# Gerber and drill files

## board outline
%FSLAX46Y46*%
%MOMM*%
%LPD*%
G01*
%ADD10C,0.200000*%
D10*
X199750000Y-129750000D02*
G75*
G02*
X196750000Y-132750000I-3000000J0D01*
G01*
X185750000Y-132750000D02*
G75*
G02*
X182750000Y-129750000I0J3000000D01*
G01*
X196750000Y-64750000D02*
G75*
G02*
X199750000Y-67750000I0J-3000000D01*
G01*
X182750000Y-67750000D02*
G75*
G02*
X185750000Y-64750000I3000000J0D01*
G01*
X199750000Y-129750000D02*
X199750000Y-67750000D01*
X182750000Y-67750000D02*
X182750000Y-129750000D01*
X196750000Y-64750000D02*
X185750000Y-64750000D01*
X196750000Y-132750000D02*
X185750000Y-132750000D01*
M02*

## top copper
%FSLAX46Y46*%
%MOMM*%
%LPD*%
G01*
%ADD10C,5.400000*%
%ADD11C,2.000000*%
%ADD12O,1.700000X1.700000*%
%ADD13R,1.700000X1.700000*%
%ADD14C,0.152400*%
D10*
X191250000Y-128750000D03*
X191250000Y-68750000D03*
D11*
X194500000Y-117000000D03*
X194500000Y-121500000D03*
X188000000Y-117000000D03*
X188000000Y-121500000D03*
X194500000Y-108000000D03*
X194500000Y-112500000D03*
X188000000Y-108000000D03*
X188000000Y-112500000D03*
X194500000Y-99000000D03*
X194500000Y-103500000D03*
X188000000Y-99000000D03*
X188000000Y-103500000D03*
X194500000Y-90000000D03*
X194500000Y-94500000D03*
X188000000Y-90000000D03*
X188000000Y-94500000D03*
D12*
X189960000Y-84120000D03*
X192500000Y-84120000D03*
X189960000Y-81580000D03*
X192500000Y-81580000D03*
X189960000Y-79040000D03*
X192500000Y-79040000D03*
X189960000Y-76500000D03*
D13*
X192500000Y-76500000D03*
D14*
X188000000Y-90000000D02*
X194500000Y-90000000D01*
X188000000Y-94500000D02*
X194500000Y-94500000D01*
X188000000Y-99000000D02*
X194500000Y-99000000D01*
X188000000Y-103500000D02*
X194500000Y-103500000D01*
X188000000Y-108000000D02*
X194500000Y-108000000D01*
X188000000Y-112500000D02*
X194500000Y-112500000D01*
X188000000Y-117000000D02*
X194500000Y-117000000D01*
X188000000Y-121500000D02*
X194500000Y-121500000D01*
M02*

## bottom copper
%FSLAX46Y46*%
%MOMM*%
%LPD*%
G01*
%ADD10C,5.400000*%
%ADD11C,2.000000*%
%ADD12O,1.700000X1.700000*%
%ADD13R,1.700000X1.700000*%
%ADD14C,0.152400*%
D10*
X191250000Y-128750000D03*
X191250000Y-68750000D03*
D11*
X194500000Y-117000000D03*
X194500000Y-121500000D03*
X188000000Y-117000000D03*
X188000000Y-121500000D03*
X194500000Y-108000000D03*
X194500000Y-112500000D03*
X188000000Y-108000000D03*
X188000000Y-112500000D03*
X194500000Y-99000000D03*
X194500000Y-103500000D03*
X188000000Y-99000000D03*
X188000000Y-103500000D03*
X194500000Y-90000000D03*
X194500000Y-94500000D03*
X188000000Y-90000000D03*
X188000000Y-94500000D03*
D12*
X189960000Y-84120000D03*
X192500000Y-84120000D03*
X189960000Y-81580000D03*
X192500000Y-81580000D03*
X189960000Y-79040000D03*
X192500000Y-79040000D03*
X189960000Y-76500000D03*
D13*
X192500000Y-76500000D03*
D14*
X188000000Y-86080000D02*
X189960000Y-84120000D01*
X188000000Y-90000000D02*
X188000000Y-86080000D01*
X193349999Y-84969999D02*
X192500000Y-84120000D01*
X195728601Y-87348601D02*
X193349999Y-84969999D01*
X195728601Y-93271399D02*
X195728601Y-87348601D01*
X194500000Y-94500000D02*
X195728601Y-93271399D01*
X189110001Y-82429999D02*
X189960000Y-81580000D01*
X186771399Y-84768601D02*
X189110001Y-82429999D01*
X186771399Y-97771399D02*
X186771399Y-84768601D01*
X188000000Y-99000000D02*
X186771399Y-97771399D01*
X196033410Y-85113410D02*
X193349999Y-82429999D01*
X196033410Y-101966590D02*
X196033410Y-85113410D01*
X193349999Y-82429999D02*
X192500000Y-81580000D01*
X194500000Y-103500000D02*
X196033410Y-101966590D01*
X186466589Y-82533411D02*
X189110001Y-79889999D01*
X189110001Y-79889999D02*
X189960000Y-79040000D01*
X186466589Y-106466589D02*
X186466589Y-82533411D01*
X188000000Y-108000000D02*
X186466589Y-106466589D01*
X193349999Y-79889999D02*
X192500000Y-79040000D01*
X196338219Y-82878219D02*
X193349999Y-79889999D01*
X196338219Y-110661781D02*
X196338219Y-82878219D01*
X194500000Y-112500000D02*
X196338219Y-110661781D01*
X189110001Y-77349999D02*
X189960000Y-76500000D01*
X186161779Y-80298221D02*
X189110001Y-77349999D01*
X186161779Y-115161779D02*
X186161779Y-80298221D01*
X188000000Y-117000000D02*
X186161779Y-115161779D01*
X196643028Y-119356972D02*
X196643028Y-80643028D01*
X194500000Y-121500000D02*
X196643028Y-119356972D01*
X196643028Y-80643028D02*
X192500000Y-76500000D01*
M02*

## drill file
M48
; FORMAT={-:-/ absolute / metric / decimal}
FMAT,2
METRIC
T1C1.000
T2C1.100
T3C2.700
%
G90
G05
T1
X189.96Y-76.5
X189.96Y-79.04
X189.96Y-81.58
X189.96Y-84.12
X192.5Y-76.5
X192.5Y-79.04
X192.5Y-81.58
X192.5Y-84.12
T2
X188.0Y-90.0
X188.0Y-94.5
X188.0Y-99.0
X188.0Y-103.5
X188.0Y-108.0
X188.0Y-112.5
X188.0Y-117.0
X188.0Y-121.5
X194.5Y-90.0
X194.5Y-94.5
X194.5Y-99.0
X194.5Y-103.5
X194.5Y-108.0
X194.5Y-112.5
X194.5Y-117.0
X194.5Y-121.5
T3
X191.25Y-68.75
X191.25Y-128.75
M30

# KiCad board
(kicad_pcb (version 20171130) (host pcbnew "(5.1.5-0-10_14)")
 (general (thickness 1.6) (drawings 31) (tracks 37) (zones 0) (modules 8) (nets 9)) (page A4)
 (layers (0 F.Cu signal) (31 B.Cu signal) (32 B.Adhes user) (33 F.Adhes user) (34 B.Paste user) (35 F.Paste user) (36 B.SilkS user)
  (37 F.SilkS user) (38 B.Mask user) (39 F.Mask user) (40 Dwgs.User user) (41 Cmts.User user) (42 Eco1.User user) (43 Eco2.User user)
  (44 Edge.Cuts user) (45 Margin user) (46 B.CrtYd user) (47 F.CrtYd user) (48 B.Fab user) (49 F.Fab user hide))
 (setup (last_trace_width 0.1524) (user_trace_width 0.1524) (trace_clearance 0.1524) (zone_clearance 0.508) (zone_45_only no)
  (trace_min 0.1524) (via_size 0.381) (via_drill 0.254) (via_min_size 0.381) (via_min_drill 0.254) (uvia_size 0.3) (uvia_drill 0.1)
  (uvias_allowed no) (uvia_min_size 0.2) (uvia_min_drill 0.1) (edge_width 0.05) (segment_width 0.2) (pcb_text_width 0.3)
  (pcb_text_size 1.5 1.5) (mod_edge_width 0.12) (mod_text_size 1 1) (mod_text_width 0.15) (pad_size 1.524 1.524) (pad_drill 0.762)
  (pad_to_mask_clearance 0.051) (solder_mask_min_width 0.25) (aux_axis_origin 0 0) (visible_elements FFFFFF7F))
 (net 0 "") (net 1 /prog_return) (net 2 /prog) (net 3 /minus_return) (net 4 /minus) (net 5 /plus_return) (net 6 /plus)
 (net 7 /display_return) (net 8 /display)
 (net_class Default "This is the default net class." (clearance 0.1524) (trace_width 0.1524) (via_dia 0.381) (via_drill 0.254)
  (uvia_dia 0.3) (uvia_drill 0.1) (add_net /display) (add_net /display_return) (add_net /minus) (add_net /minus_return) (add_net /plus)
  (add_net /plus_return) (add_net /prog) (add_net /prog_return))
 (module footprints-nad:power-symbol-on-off (layer F.Cu) (at 185.25 92.25 270)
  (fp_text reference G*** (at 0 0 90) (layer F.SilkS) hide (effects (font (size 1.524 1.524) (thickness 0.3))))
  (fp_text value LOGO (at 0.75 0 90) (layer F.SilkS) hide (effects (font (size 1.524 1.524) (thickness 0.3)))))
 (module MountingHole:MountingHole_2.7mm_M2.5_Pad (layer F.Cu) (at 191.25 128.75)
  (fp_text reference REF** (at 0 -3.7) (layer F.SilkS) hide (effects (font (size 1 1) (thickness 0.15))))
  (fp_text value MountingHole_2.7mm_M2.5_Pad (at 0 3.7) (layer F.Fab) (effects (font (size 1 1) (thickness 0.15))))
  (pad 1 thru_hole circle (at 0 0) (size 5.4 5.4) (drill 2.7) (layers *.Cu *.Mask)))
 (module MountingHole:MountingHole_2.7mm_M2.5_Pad (layer F.Cu) (at 191.25 68.75)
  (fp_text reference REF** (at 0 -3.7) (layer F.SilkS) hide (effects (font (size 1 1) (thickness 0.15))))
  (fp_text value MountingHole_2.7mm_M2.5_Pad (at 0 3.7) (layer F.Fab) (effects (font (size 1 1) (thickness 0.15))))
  (pad 1 thru_hole circle (at 0 0) (size 5.4 5.4) (drill 2.7) (layers *.Cu *.Mask)))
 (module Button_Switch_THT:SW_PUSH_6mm (layer F.Cu) (at 188 117)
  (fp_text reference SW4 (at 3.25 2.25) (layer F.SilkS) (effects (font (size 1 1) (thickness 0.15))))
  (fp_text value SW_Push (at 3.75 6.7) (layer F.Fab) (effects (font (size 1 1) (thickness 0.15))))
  (pad 1 thru_hole circle (at 6.5 0 90) (size 2 2) (drill 1.1) (layers *.Cu *.Mask) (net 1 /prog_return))
  (pad 2 thru_hole circle (at 6.5 4.5 90) (size 2 2) (drill 1.1) (layers *.Cu *.Mask) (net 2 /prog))
  (pad 1 thru_hole circle (at 0 0 90) (size 2 2) (drill 1.1) (layers *.Cu *.Mask) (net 1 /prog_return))
  (pad 2 thru_hole circle (at 0 4.5 90) (size 2 2) (drill 1.1) (layers *.Cu *.Mask) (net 2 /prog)))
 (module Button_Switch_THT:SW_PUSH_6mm (layer F.Cu) (at 188 108)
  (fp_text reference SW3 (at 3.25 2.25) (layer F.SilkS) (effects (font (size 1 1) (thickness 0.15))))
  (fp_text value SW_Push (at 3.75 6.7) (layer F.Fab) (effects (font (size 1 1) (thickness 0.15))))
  (pad 1 thru_hole circle (at 6.5 0 90) (size 2 2) (drill 1.1) (layers *.Cu *.Mask) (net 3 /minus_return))
  (pad 2 thru_hole circle (at 6.5 4.5 90) (size 2 2) (drill 1.1) (layers *.Cu *.Mask) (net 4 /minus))
  (pad 1 thru_hole circle (at 0 0 90) (size 2 2) (drill 1.1) (layers *.Cu *.Mask) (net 3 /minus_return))
  (pad 2 thru_hole circle (at 0 4.5 90) (size 2 2) (drill 1.1) (layers *.Cu *.Mask) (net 4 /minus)))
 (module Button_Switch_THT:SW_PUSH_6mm (layer F.Cu) (at 188 99)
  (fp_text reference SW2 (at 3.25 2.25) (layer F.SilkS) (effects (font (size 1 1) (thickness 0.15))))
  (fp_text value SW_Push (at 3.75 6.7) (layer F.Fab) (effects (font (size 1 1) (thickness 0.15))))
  (pad 1 thru_hole circle (at 6.5 0 90) (size 2 2) (drill 1.1) (layers *.Cu *.Mask) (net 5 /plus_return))
  (pad 2 thru_hole circle (at 6.5 4.5 90) (size 2 2) (drill 1.1) (layers *.Cu *.Mask) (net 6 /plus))
  (pad 1 thru_hole circle (at 0 0 90) (size 2 2) (drill 1.1) (layers *.Cu *.Mask) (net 5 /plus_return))
  (pad 2 thru_hole circle (at 0 4.5 90) (size 2 2) (drill 1.1) (layers *.Cu *.Mask) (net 6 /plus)))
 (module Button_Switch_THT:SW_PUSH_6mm (layer F.Cu) (at 188 90)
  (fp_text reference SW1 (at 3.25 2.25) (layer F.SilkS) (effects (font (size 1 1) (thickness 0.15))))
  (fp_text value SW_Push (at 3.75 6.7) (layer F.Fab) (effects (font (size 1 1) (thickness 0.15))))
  (pad 1 thru_hole circle (at 6.5 0 90) (size 2 2) (drill 1.1) (layers *.Cu *.Mask) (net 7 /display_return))
  (pad 2 thru_hole circle (at 6.5 4.5 90) (size 2 2) (drill 1.1) (layers *.Cu *.Mask) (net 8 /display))
  (pad 1 thru_hole circle (at 0 0 90) (size 2 2) (drill 1.1) (layers *.Cu *.Mask) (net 7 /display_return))
  (pad 2 thru_hole circle (at 0 4.5 90) (size 2 2) (drill 1.1) (layers *.Cu *.Mask) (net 8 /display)))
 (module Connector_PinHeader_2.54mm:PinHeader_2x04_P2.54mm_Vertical (layer B.Cu) (at 192.5 76.5 180)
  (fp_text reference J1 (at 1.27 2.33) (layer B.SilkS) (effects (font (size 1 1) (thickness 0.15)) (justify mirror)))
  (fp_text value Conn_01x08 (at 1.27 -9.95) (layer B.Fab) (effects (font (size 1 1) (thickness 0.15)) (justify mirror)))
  (pad 8 thru_hole oval (at 2.54 -7.62 180) (size 1.7 1.7) (drill 1) (layers *.Cu *.Mask) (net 7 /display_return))
  (pad 7 thru_hole oval (at 0 -7.62 180) (size 1.7 1.7) (drill 1) (layers *.Cu *.Mask) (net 8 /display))
  (pad 6 thru_hole oval (at 2.54 -5.08 180) (size 1.7 1.7) (drill 1) (layers *.Cu *.Mask) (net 5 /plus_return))
  (pad 5 thru_hole oval (at 0 -5.08 180) (size 1.7 1.7) (drill 1) (layers *.Cu *.Mask) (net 6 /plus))
  (pad 4 thru_hole oval (at 2.54 -2.54 180) (size 1.7 1.7) (drill 1) (layers *.Cu *.Mask) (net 3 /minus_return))
  (pad 3 thru_hole oval (at 0 -2.54 180) (size 1.7 1.7) (drill 1) (layers *.Cu *.Mask) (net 4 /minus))
  (pad 2 thru_hole oval (at 2.54 0 180) (size 1.7 1.7) (drill 1) (layers *.Cu *.Mask) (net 1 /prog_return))
  (pad 1 thru_hole rect (at 0 0 180) (size 1.7 1.7) (drill 1) (layers *.Cu *.Mask) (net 2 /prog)))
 (gr_arc (start 196.75 129.75) (end 196.75 132.75) (angle -90) (layer Edge.Cuts) (width 0.2))
 (gr_arc (start 185.75 129.75) (end 182.75 129.75) (angle -90) (layer Edge.Cuts) (width 0.2))
 (gr_arc (start 196.75 67.75) (end 199.75 67.75) (angle -90) (layer Edge.Cuts) (width 0.2))
 (gr_arc (start 185.75 67.75) (end 185.75 64.75) (angle -90) (layer Edge.Cuts) (width 0.2))
 (gr_line (start 199.75 129.75) (end 199.75 67.75) (layer Edge.Cuts) (width 0.2))
 (gr_line (start 182.75 67.75) (end 182.75 129.75) (layer Edge.Cuts) (width 0.2))
 (gr_line (start 196.75 64.75) (end 185.75 64.75) (layer Edge.Cuts) (width 0.2))
 (gr_line (start 196.75 132.75) (end 185.75 132.75) (layer Edge.Cuts) (width 0.2))
 (segment (start 188 90) (end 194.5 90) (width 0.1524) (layer F.Cu) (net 7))
 (segment (start 188 86.08) (end 189.96 84.12) (width 0.1524) (layer B.Cu) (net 7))
 (segment (start 188 90) (end 188 86.08) (width 0.1524) (layer B.Cu) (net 7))
 (segment (start 188 94.5) (end 194.5 94.5) (width 0.1524) (layer F.Cu) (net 8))
 (segment (start 193.349999 84.969999) (end 192.5 84.12) (width 0.1524) (layer B.Cu) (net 8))
 (segment (start 195.728601 87.348601) (end 193.349999 84.969999) (width 0.1524) (layer B.Cu) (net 8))
 (segment (start 195.728601 93.271399) (end 195.728601 87.348601) (width 0.1524) (layer B.Cu) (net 8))
 (segment (start 194.5 94.5) (end 195.728601 93.271399) (width 0.1524) (layer B.Cu) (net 8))
 (segment (start 188 99) (end 194.5 99) (width 0.1524) (layer F.Cu) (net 5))
 (segment (start 189.110001 82.429999) (end 189.96 81.58) (width 0.1524) (layer B.Cu) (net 5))
 (segment (start 186.771399 84.768601) (end 189.110001 82.429999) (width 0.1524) (layer B.Cu) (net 5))
 (segment (start 186.771399 97.771399) (end 186.771399 84.768601) (width 0.1524) (layer B.Cu) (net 5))
 (segment (start 188 99) (end 186.771399 97.771399) (width 0.1524) (layer B.Cu) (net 5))
 (segment (start 188 103.5) (end 194.5 103.5) (width 0.1524) (layer F.Cu) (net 6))
 (segment (start 196.03341 85.11341) (end 193.349999 82.429999) (width 0.1524) (layer B.Cu) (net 6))
 (segment (start 196.03341 101.96659) (end 196.03341 85.11341) (width 0.1524) (layer B.Cu) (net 6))
 (segment (start 193.349999 82.429999) (end 192.5 81.58) (width 0.1524) (layer B.Cu) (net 6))
 (segment (start 194.5 103.5) (end 196.03341 101.96659) (width 0.1524) (layer B.Cu) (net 6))
 (segment (start 188 108) (end 194.5 108) (width 0.1524) (layer F.Cu) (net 3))
 (segment (start 186.466589 82.533411) (end 189.110001 79.889999) (width 0.1524) (layer B.Cu) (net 3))
 (segment (start 189.110001 79.889999) (end 189.96 79.04) (width 0.1524) (layer B.Cu) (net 3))
 (segment (start 186.466589 106.466589) (end 186.466589 82.533411) (width 0.1524) (layer B.Cu) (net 3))
 (segment (start 188 108) (end 186.466589 106.466589) (width 0.1524) (layer B.Cu) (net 3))
 (segment (start 188 112.5) (end 194.5 112.5) (width 0.1524) (layer F.Cu) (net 4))
 (segment (start 193.349999 79.889999) (end 192.5 79.04) (width 0.1524) (layer B.Cu) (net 4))
 (segment (start 196.338219 82.878219) (end 193.349999 79.889999) (width 0.1524) (layer B.Cu) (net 4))
 (segment (start 196.338219 110.661781) (end 196.338219 82.878219) (width 0.1524) (layer B.Cu) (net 4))
 (segment (start 194.5 112.5) (end 196.338219 110.661781) (width 0.1524) (layer B.Cu) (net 4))
 (segment (start 188 117) (end 194.5 117) (width 0.1524) (layer F.Cu) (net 1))
 (segment (start 189.110001 77.349999) (end 189.96 76.5) (width 0.1524) (layer B.Cu) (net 1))
 (segment (start 186.161779 80.298221) (end 189.110001 77.349999) (width 0.1524) (layer B.Cu) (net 1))
 (segment (start 186.161779 115.161779) (end 186.161779 80.298221) (width 0.1524) (layer B.Cu) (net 1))
 (segment (start 188 117) (end 186.161779 115.161779) (width 0.1524) (layer B.Cu) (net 1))
 (segment (start 188 121.5) (end 194.5 121.5) (width 0.1524) (layer F.Cu) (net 2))
 (segment (start 196.643028 119.356972) (end 196.643028 80.643028) (width 0.1524) (layer B.Cu) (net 2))
 (segment (start 194.5 121.5) (end 196.643028 119.356972) (width 0.1524) (layer B.Cu) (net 2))
 (segment (start 196.643028 80.643028) (end 192.5 76.5) (width 0.1524) (layer B.Cu) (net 2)))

